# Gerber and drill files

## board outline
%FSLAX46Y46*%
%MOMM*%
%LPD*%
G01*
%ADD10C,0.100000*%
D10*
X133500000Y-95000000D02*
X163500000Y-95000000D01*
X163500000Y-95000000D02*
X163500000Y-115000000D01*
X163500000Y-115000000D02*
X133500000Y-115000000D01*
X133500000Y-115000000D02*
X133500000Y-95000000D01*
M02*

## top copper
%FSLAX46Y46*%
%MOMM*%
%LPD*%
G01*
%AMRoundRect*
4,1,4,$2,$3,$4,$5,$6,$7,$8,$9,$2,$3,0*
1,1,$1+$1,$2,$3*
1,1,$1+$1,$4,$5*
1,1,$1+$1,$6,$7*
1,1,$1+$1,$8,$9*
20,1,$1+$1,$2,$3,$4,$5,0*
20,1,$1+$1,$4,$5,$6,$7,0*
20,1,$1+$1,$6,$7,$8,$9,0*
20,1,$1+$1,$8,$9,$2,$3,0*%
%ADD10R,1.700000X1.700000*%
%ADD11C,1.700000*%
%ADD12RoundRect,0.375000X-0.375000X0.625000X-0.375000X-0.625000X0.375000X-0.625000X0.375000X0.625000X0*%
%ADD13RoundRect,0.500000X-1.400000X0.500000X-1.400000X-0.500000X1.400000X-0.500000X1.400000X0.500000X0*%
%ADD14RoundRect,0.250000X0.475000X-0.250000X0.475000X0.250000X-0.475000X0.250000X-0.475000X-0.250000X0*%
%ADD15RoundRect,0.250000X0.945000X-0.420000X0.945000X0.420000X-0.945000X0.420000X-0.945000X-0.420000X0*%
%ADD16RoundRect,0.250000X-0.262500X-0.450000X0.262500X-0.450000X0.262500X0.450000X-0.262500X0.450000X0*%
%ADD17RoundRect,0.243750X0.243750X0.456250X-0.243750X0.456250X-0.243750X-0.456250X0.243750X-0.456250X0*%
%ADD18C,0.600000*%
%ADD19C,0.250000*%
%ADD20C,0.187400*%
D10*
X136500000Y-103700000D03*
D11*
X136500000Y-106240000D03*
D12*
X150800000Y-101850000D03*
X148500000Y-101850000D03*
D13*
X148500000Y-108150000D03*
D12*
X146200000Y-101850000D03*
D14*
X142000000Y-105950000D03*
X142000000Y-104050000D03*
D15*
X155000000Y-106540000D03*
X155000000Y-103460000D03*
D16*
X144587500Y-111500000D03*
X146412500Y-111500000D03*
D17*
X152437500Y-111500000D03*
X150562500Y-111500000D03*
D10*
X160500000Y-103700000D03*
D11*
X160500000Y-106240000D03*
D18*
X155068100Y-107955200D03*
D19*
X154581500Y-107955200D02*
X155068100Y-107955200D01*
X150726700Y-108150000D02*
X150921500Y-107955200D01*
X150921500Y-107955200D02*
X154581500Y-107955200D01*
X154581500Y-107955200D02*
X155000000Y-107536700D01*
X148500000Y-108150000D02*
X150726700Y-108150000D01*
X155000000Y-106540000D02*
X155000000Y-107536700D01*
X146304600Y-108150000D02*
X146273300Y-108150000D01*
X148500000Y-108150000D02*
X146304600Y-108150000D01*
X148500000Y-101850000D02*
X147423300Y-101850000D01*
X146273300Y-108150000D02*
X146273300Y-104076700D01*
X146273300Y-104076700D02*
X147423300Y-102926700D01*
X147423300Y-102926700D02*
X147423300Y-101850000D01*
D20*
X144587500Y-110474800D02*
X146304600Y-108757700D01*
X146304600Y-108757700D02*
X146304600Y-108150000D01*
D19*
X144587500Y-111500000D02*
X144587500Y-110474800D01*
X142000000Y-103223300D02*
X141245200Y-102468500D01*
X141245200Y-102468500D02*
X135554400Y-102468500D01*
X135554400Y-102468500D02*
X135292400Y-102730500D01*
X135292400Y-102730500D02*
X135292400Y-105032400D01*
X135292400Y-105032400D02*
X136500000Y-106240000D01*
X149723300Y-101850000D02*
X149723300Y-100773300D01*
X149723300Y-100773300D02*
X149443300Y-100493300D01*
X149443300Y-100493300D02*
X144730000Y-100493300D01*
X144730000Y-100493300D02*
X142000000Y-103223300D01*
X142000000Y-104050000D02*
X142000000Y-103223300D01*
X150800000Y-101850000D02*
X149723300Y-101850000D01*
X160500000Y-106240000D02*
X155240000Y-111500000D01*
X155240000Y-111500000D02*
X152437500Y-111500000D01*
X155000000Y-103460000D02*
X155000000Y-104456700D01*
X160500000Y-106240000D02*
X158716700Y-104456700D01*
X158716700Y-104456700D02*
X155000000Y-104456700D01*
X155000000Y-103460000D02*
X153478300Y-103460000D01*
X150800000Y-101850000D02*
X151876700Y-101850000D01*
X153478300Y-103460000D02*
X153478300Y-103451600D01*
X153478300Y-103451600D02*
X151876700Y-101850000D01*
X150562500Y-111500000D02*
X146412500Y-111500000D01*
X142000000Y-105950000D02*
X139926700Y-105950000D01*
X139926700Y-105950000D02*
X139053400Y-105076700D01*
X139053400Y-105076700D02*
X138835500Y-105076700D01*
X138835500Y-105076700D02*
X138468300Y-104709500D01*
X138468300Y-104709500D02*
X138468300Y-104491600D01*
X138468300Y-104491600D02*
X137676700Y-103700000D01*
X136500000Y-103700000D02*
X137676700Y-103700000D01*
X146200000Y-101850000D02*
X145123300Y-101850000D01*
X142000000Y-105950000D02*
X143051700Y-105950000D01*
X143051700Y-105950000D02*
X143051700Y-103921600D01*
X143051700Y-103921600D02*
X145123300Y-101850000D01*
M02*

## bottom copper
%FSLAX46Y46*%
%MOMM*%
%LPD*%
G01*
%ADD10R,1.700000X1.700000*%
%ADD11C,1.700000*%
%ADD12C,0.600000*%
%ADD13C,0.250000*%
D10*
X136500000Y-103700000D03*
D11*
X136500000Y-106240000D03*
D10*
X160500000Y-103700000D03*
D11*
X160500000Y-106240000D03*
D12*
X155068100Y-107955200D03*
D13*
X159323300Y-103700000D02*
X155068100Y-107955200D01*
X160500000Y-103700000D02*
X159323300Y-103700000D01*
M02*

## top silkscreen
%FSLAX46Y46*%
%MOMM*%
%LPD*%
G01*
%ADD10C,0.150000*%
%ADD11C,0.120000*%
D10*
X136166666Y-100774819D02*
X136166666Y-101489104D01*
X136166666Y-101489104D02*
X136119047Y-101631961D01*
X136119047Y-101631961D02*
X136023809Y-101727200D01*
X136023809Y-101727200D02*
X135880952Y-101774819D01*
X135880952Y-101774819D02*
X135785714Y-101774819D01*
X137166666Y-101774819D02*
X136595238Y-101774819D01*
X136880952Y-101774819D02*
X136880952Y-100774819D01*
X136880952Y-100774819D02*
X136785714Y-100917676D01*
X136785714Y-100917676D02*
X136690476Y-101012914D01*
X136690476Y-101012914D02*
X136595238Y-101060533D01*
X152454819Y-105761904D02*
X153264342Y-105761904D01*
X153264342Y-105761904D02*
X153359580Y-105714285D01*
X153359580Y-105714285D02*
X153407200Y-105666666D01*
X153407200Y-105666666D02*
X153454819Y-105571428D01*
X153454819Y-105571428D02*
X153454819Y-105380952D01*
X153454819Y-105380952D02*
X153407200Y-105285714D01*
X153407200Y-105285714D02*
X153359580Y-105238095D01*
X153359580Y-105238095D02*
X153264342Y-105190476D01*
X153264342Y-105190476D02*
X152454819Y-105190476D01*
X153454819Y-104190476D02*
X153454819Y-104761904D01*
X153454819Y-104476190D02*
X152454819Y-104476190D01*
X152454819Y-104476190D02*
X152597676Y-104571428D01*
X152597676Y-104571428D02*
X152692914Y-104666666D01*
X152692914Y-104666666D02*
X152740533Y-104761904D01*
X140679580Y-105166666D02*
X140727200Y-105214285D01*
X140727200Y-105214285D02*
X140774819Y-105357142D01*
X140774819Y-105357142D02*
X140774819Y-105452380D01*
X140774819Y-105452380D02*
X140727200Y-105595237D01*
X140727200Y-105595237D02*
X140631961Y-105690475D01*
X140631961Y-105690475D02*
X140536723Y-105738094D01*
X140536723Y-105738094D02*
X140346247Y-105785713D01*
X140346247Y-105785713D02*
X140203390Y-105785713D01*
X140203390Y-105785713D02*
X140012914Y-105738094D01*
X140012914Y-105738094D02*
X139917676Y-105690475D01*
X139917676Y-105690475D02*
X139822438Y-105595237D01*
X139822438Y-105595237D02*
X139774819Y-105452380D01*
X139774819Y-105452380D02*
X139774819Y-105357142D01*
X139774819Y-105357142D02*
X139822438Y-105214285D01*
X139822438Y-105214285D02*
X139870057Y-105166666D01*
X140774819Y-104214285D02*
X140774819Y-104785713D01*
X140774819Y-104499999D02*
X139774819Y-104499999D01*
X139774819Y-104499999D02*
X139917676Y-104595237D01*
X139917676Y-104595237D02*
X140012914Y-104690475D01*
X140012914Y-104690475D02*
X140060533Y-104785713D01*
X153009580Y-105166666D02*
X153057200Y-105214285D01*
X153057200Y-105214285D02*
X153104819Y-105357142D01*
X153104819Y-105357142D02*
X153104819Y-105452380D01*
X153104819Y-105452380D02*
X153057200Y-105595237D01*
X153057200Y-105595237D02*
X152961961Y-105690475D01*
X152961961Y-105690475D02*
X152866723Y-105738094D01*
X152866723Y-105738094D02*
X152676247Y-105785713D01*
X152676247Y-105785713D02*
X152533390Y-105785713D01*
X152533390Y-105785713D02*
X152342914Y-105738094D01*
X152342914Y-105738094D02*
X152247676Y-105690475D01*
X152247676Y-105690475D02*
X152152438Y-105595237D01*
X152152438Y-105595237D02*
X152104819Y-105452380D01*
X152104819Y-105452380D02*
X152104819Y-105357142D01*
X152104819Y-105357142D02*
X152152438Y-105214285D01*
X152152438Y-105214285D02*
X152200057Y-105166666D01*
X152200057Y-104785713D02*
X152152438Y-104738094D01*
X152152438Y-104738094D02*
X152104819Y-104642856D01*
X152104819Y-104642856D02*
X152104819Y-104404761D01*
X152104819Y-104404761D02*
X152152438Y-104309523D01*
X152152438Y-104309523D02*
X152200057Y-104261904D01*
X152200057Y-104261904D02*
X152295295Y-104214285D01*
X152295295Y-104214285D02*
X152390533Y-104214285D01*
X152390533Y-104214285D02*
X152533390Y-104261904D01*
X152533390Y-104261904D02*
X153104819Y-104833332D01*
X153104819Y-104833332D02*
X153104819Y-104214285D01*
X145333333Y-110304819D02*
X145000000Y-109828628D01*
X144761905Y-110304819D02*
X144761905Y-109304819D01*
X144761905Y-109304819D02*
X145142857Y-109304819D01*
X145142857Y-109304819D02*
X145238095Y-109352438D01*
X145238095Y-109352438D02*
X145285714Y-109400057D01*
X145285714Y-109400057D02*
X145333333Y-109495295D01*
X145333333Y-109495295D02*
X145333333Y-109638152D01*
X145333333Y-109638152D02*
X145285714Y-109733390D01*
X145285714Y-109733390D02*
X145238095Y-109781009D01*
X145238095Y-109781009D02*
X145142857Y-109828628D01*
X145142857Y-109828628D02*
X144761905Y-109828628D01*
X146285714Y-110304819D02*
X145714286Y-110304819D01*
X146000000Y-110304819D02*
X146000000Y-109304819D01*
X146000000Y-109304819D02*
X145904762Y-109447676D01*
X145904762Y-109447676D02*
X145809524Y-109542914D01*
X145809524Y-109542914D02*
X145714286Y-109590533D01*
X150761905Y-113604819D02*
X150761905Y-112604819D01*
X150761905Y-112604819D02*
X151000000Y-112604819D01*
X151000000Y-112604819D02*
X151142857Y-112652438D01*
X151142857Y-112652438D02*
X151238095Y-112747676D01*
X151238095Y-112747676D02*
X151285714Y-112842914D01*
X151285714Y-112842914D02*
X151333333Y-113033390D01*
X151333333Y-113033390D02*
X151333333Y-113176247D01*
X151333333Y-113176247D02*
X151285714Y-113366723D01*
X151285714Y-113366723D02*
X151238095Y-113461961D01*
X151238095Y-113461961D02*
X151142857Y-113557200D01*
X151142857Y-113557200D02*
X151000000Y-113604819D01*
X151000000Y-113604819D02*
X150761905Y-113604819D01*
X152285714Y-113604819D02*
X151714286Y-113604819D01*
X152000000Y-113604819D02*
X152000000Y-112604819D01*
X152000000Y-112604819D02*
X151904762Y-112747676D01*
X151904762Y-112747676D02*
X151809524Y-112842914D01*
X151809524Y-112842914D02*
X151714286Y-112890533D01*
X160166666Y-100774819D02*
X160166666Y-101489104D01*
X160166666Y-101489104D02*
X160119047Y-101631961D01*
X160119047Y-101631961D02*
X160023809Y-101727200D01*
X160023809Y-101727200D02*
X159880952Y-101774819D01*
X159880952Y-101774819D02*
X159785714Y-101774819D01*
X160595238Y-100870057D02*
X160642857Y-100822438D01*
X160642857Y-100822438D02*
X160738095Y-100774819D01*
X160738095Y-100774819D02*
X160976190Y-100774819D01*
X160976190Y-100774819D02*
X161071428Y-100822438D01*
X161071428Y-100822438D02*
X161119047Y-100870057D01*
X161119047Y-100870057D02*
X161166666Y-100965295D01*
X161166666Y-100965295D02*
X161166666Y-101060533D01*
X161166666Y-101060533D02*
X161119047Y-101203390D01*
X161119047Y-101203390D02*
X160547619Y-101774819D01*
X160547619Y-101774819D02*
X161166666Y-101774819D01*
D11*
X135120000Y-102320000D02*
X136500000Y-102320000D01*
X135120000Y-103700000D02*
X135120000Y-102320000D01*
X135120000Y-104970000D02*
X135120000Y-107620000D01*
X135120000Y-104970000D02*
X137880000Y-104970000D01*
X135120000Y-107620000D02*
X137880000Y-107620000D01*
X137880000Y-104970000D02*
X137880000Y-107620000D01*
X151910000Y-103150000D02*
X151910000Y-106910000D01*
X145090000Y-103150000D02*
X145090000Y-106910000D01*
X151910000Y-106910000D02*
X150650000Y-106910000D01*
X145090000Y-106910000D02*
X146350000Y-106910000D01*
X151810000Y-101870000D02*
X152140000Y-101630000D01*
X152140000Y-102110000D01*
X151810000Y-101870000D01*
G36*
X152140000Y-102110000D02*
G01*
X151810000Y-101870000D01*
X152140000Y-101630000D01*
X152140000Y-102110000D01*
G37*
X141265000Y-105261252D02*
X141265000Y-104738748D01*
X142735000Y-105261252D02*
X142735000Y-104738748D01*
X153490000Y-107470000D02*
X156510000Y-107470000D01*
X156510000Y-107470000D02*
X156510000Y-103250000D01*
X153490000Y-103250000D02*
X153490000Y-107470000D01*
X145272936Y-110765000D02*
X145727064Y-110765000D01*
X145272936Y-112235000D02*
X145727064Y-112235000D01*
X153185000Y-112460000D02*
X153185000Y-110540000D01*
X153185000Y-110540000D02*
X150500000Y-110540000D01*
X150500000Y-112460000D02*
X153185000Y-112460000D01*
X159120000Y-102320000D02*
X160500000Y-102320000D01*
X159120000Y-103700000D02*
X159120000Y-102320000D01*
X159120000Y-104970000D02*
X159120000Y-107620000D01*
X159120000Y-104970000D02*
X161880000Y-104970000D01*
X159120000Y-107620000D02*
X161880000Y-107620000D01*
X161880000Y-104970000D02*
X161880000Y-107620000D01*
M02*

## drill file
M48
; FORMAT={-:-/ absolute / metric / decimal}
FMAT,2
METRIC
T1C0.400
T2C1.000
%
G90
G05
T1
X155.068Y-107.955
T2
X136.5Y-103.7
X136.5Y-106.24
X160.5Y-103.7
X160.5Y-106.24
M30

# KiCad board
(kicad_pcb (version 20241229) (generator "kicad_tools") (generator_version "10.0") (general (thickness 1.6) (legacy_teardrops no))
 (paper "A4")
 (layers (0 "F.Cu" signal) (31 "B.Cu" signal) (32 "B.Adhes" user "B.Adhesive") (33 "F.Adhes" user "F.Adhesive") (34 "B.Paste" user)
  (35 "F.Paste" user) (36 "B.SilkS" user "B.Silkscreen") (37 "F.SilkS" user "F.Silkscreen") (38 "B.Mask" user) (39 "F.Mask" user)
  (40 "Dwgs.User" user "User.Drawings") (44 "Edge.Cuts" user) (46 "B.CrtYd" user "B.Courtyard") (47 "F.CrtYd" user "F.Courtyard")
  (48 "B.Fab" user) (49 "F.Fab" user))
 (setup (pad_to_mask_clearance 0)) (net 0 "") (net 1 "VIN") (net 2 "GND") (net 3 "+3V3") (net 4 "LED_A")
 (gr_line (start 133.5 95) (end 163.5 95) (stroke (width 0.1) (type default)) (layer "Edge.Cuts"))
 (gr_line (start 163.5 95) (end 163.5 115) (stroke (width 0.1) (type default)) (layer "Edge.Cuts"))
 (gr_line (start 163.5 115) (end 133.5 115) (stroke (width 0.1) (type default)) (layer "Edge.Cuts"))
 (gr_line (start 133.5 115) (end 133.5 95) (stroke (width 0.1) (type default)) (layer "Edge.Cuts"))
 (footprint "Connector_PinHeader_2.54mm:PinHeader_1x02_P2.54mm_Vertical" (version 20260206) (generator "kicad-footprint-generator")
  (layer "F.Cu") (at 136.5 103.7)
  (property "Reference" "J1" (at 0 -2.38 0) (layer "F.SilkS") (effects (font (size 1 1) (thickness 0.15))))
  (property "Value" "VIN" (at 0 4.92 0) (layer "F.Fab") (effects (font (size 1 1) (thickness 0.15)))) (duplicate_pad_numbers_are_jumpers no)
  (fp_line (start -1.38 -1.38) (end 0 -1.38) (stroke (width 0.12) (type solid)) (layer "F.SilkS"))
  (fp_line (start -1.38 0) (end -1.38 -1.38) (stroke (width 0.12) (type solid)) (layer "F.SilkS"))
  (fp_line (start -1.38 1.27) (end -1.38 3.92) (stroke (width 0.12) (type solid)) (layer "F.SilkS"))
  (fp_line (start -1.38 1.27) (end 1.38 1.27) (stroke (width 0.12) (type solid)) (layer "F.SilkS"))
  (fp_line (start -1.38 3.92) (end 1.38 3.92) (stroke (width 0.12) (type solid)) (layer "F.SilkS"))
  (fp_line (start 1.38 1.27) (end 1.38 3.92) (stroke (width 0.12) (type solid)) (layer "F.SilkS"))
  (pad "1" thru_hole rect (at 0 0) (size 1.7 1.7) (drill 1) (layers "*.Cu" "*.Mask") (remove_unused_layers no) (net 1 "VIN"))
  (pad "2" thru_hole circle (at 0 2.54) (size 1.7 1.7) (drill 1) (layers "*.Cu" "*.Mask") (remove_unused_layers no) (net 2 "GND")))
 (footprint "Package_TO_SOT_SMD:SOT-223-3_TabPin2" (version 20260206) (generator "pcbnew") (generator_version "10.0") (layer "F.Cu")
  (at 148.5 105 -90)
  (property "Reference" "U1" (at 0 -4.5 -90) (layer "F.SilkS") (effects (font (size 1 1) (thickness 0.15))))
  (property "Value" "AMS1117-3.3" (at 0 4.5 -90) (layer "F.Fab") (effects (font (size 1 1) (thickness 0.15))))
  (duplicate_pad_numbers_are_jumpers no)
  (fp_line (start -1.85 -3.41) (end 1.91 -3.41) (stroke (width 0.12) (type solid)) (layer "F.SilkS"))
  (fp_line (start -1.85 3.41) (end 1.91 3.41) (stroke (width 0.12) (type solid)) (layer "F.SilkS"))
  (fp_line (start 1.91 -3.41) (end 1.91 -2.15) (stroke (width 0.12) (type solid)) (layer "F.SilkS"))
  (fp_line (start 1.91 3.41) (end 1.91 2.15) (stroke (width 0.12) (type solid)) (layer "F.SilkS"))
  (fp_poly
   (pts (xy -3.13 -3.31) (xy -3.37 -3.64) (xy -2.89 -3.64) (xy -3.13 -3.31)) (stroke (width 0.12) (type solid)) (fill yes) (layer "F.SilkS"))
  (pad "1" smd roundrect (at -3.15 -2.3 -90) (size 2 1.5) (layers "F.Cu" "F.Mask" "F.Paste") (roundrect_rratio 0.25) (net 2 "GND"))
  (pad "2" smd roundrect (at -3.15 0 -90) (size 2 1.5) (layers "F.Cu" "F.Mask" "F.Paste") (roundrect_rratio 0.25) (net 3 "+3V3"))
  (pad "2" smd roundrect (at 3.15 0 -90) (size 2 3.8) (layers "F.Cu" "F.Mask" "F.Paste") (roundrect_rratio 0.25) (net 3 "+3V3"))
  (pad "3" smd roundrect (at -3.15 2.3 -90) (size 2 1.5) (layers "F.Cu" "F.Mask" "F.Paste") (roundrect_rratio 0.25) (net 1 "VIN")))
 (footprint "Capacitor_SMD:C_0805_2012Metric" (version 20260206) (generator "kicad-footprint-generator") (layer "F.Cu") (at 142 105 90)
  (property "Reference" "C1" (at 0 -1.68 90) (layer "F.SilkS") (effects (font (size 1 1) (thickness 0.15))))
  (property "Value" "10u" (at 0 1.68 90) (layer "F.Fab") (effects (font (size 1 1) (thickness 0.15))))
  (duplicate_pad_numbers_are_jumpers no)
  (fp_line (start -0.261252 -0.735) (end 0.261252 -0.735) (stroke (width 0.12) (type solid)) (layer "F.SilkS"))
  (fp_line (start -0.261252 0.735) (end 0.261252 0.735) (stroke (width 0.12) (type solid)) (layer "F.SilkS"))
  (pad "1" smd roundrect (at -0.95 0 90) (size 1 1.45) (layers "F.Cu" "F.Mask" "F.Paste") (roundrect_rratio 0.25) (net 1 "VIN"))
  (pad "2" smd roundrect (at 0.95 0 90) (size 1 1.45) (layers "F.Cu" "F.Mask" "F.Paste") (roundrect_rratio 0.25) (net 2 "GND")))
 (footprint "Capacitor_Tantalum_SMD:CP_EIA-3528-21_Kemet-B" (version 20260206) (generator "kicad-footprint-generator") (layer "F.Cu")
  (at 155 105 90)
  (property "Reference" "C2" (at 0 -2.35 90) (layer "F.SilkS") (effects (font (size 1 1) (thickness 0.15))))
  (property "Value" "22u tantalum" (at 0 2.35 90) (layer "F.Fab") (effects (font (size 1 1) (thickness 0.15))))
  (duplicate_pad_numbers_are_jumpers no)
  (fp_line (start -2.47 -1.51) (end -2.47 1.51) (stroke (width 0.12) (type solid)) (layer "F.SilkS"))
  (fp_line (start -2.47 1.51) (end 1.75 1.51) (stroke (width 0.12) (type solid)) (layer "F.SilkS"))
  (fp_line (start 1.75 -1.51) (end -2.47 -1.51) (stroke (width 0.12) (type solid)) (layer "F.SilkS"))
  (pad "1" smd roundrect (at -1.54 0 90) (size 1.34 2.39) (layers "F.Cu" "F.Mask" "F.Paste") (roundrect_rratio 0.186567) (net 3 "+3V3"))
  (pad "2" smd roundrect (at 1.54 0 90) (size 1.34 2.39) (layers "F.Cu" "F.Mask" "F.Paste") (roundrect_rratio 0.186567) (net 2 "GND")))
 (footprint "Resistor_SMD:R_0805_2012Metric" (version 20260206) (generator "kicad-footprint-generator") (layer "F.Cu") (at 145.5 111.5)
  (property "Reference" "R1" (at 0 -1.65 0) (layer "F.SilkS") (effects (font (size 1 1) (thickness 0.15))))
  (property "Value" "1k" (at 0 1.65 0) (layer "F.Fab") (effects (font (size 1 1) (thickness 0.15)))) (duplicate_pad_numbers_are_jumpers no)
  (fp_line (start -0.227064 -0.735) (end 0.227064 -0.735) (stroke (width 0.12) (type solid)) (layer "F.SilkS"))
  (fp_line (start -0.227064 0.735) (end 0.227064 0.735) (stroke (width 0.12) (type solid)) (layer "F.SilkS"))
  (pad "1" smd roundrect (at -0.9125 0) (size 1.025 1.4) (layers "F.Cu" "F.Mask" "F.Paste") (roundrect_rratio 0.243902) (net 3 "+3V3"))
  (pad "2" smd roundrect (at 0.9125 0) (size 1.025 1.4) (layers "F.Cu" "F.Mask" "F.Paste") (roundrect_rratio 0.243902) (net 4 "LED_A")))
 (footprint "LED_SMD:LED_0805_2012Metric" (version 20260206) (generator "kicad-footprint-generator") (layer "F.Cu") (at 151.5 111.5 180)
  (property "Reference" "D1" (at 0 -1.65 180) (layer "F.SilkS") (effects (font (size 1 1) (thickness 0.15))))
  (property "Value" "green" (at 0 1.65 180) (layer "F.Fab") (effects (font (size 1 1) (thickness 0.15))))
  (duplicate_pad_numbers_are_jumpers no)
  (fp_line (start -1.685 -0.96) (end -1.685 0.96) (stroke (width 0.12) (type solid)) (layer "F.SilkS"))
  (fp_line (start -1.685 0.96) (end 1 0.96) (stroke (width 0.12) (type solid)) (layer "F.SilkS"))
  (fp_line (start 1 -0.96) (end -1.685 -0.96) (stroke (width 0.12) (type solid)) (layer "F.SilkS"))
  (pad "1" smd roundrect (at -0.9375 0 180) (size 0.975 1.4) (layers "F.Cu" "F.Mask" "F.Paste") (roundrect_rratio 0.25) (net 2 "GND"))
  (pad "2" smd roundrect (at 0.9375 0 180) (size 0.975 1.4) (layers "F.Cu" "F.Mask" "F.Paste") (roundrect_rratio 0.25) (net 4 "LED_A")))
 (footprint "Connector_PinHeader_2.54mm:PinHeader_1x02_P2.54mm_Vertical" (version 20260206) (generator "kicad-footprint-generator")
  (layer "F.Cu") (at 160.5 103.7)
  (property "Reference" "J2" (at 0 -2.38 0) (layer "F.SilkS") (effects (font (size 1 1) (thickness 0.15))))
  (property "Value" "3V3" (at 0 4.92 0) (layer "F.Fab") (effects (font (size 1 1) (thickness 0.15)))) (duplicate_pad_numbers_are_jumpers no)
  (fp_line (start -1.38 -1.38) (end 0 -1.38) (stroke (width 0.12) (type solid)) (layer "F.SilkS"))
  (fp_line (start -1.38 0) (end -1.38 -1.38) (stroke (width 0.12) (type solid)) (layer "F.SilkS"))
  (fp_line (start -1.38 1.27) (end -1.38 3.92) (stroke (width 0.12) (type solid)) (layer "F.SilkS"))
  (fp_line (start -1.38 1.27) (end 1.38 1.27) (stroke (width 0.12) (type solid)) (layer "F.SilkS"))
  (fp_line (start -1.38 3.92) (end 1.38 3.92) (stroke (width 0.12) (type solid)) (layer "F.SilkS"))
  (fp_line (start 1.38 1.27) (end 1.38 3.92) (stroke (width 0.12) (type solid)) (layer "F.SilkS"))
  (pad "1" thru_hole rect (at 0 0) (size 1.7 1.7) (drill 1) (layers "*.Cu" "*.Mask") (remove_unused_layers no) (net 3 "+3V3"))
  (pad "2" thru_hole circle (at 0 2.54) (size 1.7 1.7) (drill 1) (layers "*.Cu" "*.Mask") (remove_unused_layers no) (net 2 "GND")))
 (segment (start 154.5815 107.9552) (end 155.0681 107.9552) (width 0.2500) (layer "F.Cu") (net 3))
 (segment (start 150.7267 108.1500) (end 150.9215 107.9552) (width 0.2500) (layer "F.Cu") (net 3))
 (segment (start 150.9215 107.9552) (end 154.5815 107.9552) (width 0.2500) (layer "F.Cu") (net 3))
 (segment (start 154.5815 107.9552) (end 155.0000 107.5367) (width 0.2500) (layer "F.Cu") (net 3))
 (segment (start 159.3233 103.7000) (end 155.0681 107.9552) (width 0.2500) (layer "B.Cu") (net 3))
 (segment (start 160.5000 103.7000) (end 159.3233 103.7000) (width 0.2500) (layer "B.Cu") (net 3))
 (segment (start 148.5000 108.1500) (end 150.7267 108.1500) (width 0.2500) (layer "F.Cu") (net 3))
 (segment (start 155.0000 106.5400) (end 155.0000 107.5367) (width 0.2500) (layer "F.Cu") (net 3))
 (segment (start 146.3046 108.1500) (end 146.2733 108.1500) (width 0.2500) (layer "F.Cu") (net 3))
 (segment (start 148.5000 108.1500) (end 146.3046 108.1500) (width 0.2500) (layer "F.Cu") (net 3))
 (segment (start 148.5000 101.8500) (end 147.4233 101.8500) (width 0.2500) (layer "F.Cu") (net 3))
 (segment (start 146.2733 108.1500) (end 146.2733 104.0767) (width 0.2500) (layer "F.Cu") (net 3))
 (segment (start 146.2733 104.0767) (end 147.4233 102.9267) (width 0.2500) (layer "F.Cu") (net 3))
 (segment (start 147.4233 102.9267) (end 147.4233 101.8500) (width 0.2500) (layer "F.Cu") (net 3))
 (segment (start 144.5875 110.4748) (end 146.3046 108.7577) (width 0.1874) (layer "F.Cu") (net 3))
 (segment (start 146.3046 108.7577) (end 146.3046 108.1500) (width 0.1874) (layer "F.Cu") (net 3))
 (segment (start 144.5875 111.5000) (end 144.5875 110.4748) (width 0.2500) (layer "F.Cu") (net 3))
 (segment (start 142.0000 103.2233) (end 141.2452 102.4685) (width 0.2500) (layer "F.Cu") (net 2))
 (segment (start 141.2452 102.4685) (end 135.5544 102.4685) (width 0.2500) (layer "F.Cu") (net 2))
 (segment (start 135.5544 102.4685) (end 135.2924 102.7305) (width 0.2500) (layer "F.Cu") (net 2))
 (segment (start 135.2924 102.7305) (end 135.2924 105.0324) (width 0.2500) (layer "F.Cu") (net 2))
 (segment (start 135.2924 105.0324) (end 136.5000 106.2400) (width 0.2500) (layer "F.Cu") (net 2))
 (segment (start 149.7233 101.8500) (end 149.7233 100.7733) (width 0.2500) (layer "F.Cu") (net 2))
 (segment (start 149.7233 100.7733) (end 149.4433 100.4933) (width 0.2500) (layer "F.Cu") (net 2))
 (segment (start 149.4433 100.4933) (end 144.7300 100.4933) (width 0.2500) (layer "F.Cu") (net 2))
 (segment (start 144.7300 100.4933) (end 142.0000 103.2233) (width 0.2500) (layer "F.Cu") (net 2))
 (segment (start 142.0000 104.0500) (end 142.0000 103.2233) (width 0.2500) (layer "F.Cu") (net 2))
 (segment (start 150.8000 101.8500) (end 149.7233 101.8500) (width 0.2500) (layer "F.Cu") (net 2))
 (segment (start 160.5000 106.2400) (end 155.2400 111.5000) (width 0.2500) (layer "F.Cu") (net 2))
 (segment (start 155.2400 111.5000) (end 152.4375 111.5000) (width 0.2500) (layer "F.Cu") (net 2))
 (segment (start 155.0000 103.4600) (end 155.0000 104.4567) (width 0.2500) (layer "F.Cu") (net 2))
 (segment (start 160.5000 106.2400) (end 158.7167 104.4567) (width 0.2500) (layer "F.Cu") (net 2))
 (segment (start 158.7167 104.4567) (end 155.0000 104.4567) (width 0.2500) (layer "F.Cu") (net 2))
 (segment (start 155.0000 103.4600) (end 153.4783 103.4600) (width 0.2500) (layer "F.Cu") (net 2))
 (segment (start 150.8000 101.8500) (end 151.8767 101.8500) (width 0.2500) (layer "F.Cu") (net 2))
 (segment (start 153.4783 103.4600) (end 153.4783 103.4516) (width 0.2500) (layer "F.Cu") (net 2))
 (segment (start 153.4783 103.4516) (end 151.8767 101.8500) (width 0.2500) (layer "F.Cu") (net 2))
 (segment (start 150.5625 111.5000) (end 146.4125 111.5000) (width 0.2500) (layer "F.Cu") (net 4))
 (segment (start 142.0000 105.9500) (end 139.9267 105.9500) (width 0.2500) (layer "F.Cu") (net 1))
 (segment (start 139.9267 105.9500) (end 139.0534 105.0767) (width 0.2500) (layer "F.Cu") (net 1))
 (segment (start 139.0534 105.0767) (end 138.8355 105.0767) (width 0.2500) (layer "F.Cu") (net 1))
 (segment (start 138.8355 105.0767) (end 138.4683 104.7095) (width 0.2500) (layer "F.Cu") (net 1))
 (segment (start 138.4683 104.7095) (end 138.4683 104.4916) (width 0.2500) (layer "F.Cu") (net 1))
 (segment (start 138.4683 104.4916) (end 137.6767 103.7000) (width 0.2500) (layer "F.Cu") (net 1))
 (segment (start 136.5000 103.7000) (end 137.6767 103.7000) (width 0.2500) (layer "F.Cu") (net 1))
 (segment (start 146.2000 101.8500) (end 145.1233 101.8500) (width 0.2500) (layer "F.Cu") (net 1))
 (segment (start 142.0000 105.9500) (end 143.0517 105.9500) (width 0.2500) (layer "F.Cu") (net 1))
 (segment (start 143.0517 105.9500) (end 143.0517 103.9216) (width 0.2500) (layer "F.Cu") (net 1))
 (segment (start 143.0517 103.9216) (end 145.1233 101.8500) (width 0.2500) (layer "F.Cu") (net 1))
 (via (at 155.0681 107.9552) (size 0.6000) (drill 0.4) (layers "F.Cu" "B.Cu") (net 3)))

